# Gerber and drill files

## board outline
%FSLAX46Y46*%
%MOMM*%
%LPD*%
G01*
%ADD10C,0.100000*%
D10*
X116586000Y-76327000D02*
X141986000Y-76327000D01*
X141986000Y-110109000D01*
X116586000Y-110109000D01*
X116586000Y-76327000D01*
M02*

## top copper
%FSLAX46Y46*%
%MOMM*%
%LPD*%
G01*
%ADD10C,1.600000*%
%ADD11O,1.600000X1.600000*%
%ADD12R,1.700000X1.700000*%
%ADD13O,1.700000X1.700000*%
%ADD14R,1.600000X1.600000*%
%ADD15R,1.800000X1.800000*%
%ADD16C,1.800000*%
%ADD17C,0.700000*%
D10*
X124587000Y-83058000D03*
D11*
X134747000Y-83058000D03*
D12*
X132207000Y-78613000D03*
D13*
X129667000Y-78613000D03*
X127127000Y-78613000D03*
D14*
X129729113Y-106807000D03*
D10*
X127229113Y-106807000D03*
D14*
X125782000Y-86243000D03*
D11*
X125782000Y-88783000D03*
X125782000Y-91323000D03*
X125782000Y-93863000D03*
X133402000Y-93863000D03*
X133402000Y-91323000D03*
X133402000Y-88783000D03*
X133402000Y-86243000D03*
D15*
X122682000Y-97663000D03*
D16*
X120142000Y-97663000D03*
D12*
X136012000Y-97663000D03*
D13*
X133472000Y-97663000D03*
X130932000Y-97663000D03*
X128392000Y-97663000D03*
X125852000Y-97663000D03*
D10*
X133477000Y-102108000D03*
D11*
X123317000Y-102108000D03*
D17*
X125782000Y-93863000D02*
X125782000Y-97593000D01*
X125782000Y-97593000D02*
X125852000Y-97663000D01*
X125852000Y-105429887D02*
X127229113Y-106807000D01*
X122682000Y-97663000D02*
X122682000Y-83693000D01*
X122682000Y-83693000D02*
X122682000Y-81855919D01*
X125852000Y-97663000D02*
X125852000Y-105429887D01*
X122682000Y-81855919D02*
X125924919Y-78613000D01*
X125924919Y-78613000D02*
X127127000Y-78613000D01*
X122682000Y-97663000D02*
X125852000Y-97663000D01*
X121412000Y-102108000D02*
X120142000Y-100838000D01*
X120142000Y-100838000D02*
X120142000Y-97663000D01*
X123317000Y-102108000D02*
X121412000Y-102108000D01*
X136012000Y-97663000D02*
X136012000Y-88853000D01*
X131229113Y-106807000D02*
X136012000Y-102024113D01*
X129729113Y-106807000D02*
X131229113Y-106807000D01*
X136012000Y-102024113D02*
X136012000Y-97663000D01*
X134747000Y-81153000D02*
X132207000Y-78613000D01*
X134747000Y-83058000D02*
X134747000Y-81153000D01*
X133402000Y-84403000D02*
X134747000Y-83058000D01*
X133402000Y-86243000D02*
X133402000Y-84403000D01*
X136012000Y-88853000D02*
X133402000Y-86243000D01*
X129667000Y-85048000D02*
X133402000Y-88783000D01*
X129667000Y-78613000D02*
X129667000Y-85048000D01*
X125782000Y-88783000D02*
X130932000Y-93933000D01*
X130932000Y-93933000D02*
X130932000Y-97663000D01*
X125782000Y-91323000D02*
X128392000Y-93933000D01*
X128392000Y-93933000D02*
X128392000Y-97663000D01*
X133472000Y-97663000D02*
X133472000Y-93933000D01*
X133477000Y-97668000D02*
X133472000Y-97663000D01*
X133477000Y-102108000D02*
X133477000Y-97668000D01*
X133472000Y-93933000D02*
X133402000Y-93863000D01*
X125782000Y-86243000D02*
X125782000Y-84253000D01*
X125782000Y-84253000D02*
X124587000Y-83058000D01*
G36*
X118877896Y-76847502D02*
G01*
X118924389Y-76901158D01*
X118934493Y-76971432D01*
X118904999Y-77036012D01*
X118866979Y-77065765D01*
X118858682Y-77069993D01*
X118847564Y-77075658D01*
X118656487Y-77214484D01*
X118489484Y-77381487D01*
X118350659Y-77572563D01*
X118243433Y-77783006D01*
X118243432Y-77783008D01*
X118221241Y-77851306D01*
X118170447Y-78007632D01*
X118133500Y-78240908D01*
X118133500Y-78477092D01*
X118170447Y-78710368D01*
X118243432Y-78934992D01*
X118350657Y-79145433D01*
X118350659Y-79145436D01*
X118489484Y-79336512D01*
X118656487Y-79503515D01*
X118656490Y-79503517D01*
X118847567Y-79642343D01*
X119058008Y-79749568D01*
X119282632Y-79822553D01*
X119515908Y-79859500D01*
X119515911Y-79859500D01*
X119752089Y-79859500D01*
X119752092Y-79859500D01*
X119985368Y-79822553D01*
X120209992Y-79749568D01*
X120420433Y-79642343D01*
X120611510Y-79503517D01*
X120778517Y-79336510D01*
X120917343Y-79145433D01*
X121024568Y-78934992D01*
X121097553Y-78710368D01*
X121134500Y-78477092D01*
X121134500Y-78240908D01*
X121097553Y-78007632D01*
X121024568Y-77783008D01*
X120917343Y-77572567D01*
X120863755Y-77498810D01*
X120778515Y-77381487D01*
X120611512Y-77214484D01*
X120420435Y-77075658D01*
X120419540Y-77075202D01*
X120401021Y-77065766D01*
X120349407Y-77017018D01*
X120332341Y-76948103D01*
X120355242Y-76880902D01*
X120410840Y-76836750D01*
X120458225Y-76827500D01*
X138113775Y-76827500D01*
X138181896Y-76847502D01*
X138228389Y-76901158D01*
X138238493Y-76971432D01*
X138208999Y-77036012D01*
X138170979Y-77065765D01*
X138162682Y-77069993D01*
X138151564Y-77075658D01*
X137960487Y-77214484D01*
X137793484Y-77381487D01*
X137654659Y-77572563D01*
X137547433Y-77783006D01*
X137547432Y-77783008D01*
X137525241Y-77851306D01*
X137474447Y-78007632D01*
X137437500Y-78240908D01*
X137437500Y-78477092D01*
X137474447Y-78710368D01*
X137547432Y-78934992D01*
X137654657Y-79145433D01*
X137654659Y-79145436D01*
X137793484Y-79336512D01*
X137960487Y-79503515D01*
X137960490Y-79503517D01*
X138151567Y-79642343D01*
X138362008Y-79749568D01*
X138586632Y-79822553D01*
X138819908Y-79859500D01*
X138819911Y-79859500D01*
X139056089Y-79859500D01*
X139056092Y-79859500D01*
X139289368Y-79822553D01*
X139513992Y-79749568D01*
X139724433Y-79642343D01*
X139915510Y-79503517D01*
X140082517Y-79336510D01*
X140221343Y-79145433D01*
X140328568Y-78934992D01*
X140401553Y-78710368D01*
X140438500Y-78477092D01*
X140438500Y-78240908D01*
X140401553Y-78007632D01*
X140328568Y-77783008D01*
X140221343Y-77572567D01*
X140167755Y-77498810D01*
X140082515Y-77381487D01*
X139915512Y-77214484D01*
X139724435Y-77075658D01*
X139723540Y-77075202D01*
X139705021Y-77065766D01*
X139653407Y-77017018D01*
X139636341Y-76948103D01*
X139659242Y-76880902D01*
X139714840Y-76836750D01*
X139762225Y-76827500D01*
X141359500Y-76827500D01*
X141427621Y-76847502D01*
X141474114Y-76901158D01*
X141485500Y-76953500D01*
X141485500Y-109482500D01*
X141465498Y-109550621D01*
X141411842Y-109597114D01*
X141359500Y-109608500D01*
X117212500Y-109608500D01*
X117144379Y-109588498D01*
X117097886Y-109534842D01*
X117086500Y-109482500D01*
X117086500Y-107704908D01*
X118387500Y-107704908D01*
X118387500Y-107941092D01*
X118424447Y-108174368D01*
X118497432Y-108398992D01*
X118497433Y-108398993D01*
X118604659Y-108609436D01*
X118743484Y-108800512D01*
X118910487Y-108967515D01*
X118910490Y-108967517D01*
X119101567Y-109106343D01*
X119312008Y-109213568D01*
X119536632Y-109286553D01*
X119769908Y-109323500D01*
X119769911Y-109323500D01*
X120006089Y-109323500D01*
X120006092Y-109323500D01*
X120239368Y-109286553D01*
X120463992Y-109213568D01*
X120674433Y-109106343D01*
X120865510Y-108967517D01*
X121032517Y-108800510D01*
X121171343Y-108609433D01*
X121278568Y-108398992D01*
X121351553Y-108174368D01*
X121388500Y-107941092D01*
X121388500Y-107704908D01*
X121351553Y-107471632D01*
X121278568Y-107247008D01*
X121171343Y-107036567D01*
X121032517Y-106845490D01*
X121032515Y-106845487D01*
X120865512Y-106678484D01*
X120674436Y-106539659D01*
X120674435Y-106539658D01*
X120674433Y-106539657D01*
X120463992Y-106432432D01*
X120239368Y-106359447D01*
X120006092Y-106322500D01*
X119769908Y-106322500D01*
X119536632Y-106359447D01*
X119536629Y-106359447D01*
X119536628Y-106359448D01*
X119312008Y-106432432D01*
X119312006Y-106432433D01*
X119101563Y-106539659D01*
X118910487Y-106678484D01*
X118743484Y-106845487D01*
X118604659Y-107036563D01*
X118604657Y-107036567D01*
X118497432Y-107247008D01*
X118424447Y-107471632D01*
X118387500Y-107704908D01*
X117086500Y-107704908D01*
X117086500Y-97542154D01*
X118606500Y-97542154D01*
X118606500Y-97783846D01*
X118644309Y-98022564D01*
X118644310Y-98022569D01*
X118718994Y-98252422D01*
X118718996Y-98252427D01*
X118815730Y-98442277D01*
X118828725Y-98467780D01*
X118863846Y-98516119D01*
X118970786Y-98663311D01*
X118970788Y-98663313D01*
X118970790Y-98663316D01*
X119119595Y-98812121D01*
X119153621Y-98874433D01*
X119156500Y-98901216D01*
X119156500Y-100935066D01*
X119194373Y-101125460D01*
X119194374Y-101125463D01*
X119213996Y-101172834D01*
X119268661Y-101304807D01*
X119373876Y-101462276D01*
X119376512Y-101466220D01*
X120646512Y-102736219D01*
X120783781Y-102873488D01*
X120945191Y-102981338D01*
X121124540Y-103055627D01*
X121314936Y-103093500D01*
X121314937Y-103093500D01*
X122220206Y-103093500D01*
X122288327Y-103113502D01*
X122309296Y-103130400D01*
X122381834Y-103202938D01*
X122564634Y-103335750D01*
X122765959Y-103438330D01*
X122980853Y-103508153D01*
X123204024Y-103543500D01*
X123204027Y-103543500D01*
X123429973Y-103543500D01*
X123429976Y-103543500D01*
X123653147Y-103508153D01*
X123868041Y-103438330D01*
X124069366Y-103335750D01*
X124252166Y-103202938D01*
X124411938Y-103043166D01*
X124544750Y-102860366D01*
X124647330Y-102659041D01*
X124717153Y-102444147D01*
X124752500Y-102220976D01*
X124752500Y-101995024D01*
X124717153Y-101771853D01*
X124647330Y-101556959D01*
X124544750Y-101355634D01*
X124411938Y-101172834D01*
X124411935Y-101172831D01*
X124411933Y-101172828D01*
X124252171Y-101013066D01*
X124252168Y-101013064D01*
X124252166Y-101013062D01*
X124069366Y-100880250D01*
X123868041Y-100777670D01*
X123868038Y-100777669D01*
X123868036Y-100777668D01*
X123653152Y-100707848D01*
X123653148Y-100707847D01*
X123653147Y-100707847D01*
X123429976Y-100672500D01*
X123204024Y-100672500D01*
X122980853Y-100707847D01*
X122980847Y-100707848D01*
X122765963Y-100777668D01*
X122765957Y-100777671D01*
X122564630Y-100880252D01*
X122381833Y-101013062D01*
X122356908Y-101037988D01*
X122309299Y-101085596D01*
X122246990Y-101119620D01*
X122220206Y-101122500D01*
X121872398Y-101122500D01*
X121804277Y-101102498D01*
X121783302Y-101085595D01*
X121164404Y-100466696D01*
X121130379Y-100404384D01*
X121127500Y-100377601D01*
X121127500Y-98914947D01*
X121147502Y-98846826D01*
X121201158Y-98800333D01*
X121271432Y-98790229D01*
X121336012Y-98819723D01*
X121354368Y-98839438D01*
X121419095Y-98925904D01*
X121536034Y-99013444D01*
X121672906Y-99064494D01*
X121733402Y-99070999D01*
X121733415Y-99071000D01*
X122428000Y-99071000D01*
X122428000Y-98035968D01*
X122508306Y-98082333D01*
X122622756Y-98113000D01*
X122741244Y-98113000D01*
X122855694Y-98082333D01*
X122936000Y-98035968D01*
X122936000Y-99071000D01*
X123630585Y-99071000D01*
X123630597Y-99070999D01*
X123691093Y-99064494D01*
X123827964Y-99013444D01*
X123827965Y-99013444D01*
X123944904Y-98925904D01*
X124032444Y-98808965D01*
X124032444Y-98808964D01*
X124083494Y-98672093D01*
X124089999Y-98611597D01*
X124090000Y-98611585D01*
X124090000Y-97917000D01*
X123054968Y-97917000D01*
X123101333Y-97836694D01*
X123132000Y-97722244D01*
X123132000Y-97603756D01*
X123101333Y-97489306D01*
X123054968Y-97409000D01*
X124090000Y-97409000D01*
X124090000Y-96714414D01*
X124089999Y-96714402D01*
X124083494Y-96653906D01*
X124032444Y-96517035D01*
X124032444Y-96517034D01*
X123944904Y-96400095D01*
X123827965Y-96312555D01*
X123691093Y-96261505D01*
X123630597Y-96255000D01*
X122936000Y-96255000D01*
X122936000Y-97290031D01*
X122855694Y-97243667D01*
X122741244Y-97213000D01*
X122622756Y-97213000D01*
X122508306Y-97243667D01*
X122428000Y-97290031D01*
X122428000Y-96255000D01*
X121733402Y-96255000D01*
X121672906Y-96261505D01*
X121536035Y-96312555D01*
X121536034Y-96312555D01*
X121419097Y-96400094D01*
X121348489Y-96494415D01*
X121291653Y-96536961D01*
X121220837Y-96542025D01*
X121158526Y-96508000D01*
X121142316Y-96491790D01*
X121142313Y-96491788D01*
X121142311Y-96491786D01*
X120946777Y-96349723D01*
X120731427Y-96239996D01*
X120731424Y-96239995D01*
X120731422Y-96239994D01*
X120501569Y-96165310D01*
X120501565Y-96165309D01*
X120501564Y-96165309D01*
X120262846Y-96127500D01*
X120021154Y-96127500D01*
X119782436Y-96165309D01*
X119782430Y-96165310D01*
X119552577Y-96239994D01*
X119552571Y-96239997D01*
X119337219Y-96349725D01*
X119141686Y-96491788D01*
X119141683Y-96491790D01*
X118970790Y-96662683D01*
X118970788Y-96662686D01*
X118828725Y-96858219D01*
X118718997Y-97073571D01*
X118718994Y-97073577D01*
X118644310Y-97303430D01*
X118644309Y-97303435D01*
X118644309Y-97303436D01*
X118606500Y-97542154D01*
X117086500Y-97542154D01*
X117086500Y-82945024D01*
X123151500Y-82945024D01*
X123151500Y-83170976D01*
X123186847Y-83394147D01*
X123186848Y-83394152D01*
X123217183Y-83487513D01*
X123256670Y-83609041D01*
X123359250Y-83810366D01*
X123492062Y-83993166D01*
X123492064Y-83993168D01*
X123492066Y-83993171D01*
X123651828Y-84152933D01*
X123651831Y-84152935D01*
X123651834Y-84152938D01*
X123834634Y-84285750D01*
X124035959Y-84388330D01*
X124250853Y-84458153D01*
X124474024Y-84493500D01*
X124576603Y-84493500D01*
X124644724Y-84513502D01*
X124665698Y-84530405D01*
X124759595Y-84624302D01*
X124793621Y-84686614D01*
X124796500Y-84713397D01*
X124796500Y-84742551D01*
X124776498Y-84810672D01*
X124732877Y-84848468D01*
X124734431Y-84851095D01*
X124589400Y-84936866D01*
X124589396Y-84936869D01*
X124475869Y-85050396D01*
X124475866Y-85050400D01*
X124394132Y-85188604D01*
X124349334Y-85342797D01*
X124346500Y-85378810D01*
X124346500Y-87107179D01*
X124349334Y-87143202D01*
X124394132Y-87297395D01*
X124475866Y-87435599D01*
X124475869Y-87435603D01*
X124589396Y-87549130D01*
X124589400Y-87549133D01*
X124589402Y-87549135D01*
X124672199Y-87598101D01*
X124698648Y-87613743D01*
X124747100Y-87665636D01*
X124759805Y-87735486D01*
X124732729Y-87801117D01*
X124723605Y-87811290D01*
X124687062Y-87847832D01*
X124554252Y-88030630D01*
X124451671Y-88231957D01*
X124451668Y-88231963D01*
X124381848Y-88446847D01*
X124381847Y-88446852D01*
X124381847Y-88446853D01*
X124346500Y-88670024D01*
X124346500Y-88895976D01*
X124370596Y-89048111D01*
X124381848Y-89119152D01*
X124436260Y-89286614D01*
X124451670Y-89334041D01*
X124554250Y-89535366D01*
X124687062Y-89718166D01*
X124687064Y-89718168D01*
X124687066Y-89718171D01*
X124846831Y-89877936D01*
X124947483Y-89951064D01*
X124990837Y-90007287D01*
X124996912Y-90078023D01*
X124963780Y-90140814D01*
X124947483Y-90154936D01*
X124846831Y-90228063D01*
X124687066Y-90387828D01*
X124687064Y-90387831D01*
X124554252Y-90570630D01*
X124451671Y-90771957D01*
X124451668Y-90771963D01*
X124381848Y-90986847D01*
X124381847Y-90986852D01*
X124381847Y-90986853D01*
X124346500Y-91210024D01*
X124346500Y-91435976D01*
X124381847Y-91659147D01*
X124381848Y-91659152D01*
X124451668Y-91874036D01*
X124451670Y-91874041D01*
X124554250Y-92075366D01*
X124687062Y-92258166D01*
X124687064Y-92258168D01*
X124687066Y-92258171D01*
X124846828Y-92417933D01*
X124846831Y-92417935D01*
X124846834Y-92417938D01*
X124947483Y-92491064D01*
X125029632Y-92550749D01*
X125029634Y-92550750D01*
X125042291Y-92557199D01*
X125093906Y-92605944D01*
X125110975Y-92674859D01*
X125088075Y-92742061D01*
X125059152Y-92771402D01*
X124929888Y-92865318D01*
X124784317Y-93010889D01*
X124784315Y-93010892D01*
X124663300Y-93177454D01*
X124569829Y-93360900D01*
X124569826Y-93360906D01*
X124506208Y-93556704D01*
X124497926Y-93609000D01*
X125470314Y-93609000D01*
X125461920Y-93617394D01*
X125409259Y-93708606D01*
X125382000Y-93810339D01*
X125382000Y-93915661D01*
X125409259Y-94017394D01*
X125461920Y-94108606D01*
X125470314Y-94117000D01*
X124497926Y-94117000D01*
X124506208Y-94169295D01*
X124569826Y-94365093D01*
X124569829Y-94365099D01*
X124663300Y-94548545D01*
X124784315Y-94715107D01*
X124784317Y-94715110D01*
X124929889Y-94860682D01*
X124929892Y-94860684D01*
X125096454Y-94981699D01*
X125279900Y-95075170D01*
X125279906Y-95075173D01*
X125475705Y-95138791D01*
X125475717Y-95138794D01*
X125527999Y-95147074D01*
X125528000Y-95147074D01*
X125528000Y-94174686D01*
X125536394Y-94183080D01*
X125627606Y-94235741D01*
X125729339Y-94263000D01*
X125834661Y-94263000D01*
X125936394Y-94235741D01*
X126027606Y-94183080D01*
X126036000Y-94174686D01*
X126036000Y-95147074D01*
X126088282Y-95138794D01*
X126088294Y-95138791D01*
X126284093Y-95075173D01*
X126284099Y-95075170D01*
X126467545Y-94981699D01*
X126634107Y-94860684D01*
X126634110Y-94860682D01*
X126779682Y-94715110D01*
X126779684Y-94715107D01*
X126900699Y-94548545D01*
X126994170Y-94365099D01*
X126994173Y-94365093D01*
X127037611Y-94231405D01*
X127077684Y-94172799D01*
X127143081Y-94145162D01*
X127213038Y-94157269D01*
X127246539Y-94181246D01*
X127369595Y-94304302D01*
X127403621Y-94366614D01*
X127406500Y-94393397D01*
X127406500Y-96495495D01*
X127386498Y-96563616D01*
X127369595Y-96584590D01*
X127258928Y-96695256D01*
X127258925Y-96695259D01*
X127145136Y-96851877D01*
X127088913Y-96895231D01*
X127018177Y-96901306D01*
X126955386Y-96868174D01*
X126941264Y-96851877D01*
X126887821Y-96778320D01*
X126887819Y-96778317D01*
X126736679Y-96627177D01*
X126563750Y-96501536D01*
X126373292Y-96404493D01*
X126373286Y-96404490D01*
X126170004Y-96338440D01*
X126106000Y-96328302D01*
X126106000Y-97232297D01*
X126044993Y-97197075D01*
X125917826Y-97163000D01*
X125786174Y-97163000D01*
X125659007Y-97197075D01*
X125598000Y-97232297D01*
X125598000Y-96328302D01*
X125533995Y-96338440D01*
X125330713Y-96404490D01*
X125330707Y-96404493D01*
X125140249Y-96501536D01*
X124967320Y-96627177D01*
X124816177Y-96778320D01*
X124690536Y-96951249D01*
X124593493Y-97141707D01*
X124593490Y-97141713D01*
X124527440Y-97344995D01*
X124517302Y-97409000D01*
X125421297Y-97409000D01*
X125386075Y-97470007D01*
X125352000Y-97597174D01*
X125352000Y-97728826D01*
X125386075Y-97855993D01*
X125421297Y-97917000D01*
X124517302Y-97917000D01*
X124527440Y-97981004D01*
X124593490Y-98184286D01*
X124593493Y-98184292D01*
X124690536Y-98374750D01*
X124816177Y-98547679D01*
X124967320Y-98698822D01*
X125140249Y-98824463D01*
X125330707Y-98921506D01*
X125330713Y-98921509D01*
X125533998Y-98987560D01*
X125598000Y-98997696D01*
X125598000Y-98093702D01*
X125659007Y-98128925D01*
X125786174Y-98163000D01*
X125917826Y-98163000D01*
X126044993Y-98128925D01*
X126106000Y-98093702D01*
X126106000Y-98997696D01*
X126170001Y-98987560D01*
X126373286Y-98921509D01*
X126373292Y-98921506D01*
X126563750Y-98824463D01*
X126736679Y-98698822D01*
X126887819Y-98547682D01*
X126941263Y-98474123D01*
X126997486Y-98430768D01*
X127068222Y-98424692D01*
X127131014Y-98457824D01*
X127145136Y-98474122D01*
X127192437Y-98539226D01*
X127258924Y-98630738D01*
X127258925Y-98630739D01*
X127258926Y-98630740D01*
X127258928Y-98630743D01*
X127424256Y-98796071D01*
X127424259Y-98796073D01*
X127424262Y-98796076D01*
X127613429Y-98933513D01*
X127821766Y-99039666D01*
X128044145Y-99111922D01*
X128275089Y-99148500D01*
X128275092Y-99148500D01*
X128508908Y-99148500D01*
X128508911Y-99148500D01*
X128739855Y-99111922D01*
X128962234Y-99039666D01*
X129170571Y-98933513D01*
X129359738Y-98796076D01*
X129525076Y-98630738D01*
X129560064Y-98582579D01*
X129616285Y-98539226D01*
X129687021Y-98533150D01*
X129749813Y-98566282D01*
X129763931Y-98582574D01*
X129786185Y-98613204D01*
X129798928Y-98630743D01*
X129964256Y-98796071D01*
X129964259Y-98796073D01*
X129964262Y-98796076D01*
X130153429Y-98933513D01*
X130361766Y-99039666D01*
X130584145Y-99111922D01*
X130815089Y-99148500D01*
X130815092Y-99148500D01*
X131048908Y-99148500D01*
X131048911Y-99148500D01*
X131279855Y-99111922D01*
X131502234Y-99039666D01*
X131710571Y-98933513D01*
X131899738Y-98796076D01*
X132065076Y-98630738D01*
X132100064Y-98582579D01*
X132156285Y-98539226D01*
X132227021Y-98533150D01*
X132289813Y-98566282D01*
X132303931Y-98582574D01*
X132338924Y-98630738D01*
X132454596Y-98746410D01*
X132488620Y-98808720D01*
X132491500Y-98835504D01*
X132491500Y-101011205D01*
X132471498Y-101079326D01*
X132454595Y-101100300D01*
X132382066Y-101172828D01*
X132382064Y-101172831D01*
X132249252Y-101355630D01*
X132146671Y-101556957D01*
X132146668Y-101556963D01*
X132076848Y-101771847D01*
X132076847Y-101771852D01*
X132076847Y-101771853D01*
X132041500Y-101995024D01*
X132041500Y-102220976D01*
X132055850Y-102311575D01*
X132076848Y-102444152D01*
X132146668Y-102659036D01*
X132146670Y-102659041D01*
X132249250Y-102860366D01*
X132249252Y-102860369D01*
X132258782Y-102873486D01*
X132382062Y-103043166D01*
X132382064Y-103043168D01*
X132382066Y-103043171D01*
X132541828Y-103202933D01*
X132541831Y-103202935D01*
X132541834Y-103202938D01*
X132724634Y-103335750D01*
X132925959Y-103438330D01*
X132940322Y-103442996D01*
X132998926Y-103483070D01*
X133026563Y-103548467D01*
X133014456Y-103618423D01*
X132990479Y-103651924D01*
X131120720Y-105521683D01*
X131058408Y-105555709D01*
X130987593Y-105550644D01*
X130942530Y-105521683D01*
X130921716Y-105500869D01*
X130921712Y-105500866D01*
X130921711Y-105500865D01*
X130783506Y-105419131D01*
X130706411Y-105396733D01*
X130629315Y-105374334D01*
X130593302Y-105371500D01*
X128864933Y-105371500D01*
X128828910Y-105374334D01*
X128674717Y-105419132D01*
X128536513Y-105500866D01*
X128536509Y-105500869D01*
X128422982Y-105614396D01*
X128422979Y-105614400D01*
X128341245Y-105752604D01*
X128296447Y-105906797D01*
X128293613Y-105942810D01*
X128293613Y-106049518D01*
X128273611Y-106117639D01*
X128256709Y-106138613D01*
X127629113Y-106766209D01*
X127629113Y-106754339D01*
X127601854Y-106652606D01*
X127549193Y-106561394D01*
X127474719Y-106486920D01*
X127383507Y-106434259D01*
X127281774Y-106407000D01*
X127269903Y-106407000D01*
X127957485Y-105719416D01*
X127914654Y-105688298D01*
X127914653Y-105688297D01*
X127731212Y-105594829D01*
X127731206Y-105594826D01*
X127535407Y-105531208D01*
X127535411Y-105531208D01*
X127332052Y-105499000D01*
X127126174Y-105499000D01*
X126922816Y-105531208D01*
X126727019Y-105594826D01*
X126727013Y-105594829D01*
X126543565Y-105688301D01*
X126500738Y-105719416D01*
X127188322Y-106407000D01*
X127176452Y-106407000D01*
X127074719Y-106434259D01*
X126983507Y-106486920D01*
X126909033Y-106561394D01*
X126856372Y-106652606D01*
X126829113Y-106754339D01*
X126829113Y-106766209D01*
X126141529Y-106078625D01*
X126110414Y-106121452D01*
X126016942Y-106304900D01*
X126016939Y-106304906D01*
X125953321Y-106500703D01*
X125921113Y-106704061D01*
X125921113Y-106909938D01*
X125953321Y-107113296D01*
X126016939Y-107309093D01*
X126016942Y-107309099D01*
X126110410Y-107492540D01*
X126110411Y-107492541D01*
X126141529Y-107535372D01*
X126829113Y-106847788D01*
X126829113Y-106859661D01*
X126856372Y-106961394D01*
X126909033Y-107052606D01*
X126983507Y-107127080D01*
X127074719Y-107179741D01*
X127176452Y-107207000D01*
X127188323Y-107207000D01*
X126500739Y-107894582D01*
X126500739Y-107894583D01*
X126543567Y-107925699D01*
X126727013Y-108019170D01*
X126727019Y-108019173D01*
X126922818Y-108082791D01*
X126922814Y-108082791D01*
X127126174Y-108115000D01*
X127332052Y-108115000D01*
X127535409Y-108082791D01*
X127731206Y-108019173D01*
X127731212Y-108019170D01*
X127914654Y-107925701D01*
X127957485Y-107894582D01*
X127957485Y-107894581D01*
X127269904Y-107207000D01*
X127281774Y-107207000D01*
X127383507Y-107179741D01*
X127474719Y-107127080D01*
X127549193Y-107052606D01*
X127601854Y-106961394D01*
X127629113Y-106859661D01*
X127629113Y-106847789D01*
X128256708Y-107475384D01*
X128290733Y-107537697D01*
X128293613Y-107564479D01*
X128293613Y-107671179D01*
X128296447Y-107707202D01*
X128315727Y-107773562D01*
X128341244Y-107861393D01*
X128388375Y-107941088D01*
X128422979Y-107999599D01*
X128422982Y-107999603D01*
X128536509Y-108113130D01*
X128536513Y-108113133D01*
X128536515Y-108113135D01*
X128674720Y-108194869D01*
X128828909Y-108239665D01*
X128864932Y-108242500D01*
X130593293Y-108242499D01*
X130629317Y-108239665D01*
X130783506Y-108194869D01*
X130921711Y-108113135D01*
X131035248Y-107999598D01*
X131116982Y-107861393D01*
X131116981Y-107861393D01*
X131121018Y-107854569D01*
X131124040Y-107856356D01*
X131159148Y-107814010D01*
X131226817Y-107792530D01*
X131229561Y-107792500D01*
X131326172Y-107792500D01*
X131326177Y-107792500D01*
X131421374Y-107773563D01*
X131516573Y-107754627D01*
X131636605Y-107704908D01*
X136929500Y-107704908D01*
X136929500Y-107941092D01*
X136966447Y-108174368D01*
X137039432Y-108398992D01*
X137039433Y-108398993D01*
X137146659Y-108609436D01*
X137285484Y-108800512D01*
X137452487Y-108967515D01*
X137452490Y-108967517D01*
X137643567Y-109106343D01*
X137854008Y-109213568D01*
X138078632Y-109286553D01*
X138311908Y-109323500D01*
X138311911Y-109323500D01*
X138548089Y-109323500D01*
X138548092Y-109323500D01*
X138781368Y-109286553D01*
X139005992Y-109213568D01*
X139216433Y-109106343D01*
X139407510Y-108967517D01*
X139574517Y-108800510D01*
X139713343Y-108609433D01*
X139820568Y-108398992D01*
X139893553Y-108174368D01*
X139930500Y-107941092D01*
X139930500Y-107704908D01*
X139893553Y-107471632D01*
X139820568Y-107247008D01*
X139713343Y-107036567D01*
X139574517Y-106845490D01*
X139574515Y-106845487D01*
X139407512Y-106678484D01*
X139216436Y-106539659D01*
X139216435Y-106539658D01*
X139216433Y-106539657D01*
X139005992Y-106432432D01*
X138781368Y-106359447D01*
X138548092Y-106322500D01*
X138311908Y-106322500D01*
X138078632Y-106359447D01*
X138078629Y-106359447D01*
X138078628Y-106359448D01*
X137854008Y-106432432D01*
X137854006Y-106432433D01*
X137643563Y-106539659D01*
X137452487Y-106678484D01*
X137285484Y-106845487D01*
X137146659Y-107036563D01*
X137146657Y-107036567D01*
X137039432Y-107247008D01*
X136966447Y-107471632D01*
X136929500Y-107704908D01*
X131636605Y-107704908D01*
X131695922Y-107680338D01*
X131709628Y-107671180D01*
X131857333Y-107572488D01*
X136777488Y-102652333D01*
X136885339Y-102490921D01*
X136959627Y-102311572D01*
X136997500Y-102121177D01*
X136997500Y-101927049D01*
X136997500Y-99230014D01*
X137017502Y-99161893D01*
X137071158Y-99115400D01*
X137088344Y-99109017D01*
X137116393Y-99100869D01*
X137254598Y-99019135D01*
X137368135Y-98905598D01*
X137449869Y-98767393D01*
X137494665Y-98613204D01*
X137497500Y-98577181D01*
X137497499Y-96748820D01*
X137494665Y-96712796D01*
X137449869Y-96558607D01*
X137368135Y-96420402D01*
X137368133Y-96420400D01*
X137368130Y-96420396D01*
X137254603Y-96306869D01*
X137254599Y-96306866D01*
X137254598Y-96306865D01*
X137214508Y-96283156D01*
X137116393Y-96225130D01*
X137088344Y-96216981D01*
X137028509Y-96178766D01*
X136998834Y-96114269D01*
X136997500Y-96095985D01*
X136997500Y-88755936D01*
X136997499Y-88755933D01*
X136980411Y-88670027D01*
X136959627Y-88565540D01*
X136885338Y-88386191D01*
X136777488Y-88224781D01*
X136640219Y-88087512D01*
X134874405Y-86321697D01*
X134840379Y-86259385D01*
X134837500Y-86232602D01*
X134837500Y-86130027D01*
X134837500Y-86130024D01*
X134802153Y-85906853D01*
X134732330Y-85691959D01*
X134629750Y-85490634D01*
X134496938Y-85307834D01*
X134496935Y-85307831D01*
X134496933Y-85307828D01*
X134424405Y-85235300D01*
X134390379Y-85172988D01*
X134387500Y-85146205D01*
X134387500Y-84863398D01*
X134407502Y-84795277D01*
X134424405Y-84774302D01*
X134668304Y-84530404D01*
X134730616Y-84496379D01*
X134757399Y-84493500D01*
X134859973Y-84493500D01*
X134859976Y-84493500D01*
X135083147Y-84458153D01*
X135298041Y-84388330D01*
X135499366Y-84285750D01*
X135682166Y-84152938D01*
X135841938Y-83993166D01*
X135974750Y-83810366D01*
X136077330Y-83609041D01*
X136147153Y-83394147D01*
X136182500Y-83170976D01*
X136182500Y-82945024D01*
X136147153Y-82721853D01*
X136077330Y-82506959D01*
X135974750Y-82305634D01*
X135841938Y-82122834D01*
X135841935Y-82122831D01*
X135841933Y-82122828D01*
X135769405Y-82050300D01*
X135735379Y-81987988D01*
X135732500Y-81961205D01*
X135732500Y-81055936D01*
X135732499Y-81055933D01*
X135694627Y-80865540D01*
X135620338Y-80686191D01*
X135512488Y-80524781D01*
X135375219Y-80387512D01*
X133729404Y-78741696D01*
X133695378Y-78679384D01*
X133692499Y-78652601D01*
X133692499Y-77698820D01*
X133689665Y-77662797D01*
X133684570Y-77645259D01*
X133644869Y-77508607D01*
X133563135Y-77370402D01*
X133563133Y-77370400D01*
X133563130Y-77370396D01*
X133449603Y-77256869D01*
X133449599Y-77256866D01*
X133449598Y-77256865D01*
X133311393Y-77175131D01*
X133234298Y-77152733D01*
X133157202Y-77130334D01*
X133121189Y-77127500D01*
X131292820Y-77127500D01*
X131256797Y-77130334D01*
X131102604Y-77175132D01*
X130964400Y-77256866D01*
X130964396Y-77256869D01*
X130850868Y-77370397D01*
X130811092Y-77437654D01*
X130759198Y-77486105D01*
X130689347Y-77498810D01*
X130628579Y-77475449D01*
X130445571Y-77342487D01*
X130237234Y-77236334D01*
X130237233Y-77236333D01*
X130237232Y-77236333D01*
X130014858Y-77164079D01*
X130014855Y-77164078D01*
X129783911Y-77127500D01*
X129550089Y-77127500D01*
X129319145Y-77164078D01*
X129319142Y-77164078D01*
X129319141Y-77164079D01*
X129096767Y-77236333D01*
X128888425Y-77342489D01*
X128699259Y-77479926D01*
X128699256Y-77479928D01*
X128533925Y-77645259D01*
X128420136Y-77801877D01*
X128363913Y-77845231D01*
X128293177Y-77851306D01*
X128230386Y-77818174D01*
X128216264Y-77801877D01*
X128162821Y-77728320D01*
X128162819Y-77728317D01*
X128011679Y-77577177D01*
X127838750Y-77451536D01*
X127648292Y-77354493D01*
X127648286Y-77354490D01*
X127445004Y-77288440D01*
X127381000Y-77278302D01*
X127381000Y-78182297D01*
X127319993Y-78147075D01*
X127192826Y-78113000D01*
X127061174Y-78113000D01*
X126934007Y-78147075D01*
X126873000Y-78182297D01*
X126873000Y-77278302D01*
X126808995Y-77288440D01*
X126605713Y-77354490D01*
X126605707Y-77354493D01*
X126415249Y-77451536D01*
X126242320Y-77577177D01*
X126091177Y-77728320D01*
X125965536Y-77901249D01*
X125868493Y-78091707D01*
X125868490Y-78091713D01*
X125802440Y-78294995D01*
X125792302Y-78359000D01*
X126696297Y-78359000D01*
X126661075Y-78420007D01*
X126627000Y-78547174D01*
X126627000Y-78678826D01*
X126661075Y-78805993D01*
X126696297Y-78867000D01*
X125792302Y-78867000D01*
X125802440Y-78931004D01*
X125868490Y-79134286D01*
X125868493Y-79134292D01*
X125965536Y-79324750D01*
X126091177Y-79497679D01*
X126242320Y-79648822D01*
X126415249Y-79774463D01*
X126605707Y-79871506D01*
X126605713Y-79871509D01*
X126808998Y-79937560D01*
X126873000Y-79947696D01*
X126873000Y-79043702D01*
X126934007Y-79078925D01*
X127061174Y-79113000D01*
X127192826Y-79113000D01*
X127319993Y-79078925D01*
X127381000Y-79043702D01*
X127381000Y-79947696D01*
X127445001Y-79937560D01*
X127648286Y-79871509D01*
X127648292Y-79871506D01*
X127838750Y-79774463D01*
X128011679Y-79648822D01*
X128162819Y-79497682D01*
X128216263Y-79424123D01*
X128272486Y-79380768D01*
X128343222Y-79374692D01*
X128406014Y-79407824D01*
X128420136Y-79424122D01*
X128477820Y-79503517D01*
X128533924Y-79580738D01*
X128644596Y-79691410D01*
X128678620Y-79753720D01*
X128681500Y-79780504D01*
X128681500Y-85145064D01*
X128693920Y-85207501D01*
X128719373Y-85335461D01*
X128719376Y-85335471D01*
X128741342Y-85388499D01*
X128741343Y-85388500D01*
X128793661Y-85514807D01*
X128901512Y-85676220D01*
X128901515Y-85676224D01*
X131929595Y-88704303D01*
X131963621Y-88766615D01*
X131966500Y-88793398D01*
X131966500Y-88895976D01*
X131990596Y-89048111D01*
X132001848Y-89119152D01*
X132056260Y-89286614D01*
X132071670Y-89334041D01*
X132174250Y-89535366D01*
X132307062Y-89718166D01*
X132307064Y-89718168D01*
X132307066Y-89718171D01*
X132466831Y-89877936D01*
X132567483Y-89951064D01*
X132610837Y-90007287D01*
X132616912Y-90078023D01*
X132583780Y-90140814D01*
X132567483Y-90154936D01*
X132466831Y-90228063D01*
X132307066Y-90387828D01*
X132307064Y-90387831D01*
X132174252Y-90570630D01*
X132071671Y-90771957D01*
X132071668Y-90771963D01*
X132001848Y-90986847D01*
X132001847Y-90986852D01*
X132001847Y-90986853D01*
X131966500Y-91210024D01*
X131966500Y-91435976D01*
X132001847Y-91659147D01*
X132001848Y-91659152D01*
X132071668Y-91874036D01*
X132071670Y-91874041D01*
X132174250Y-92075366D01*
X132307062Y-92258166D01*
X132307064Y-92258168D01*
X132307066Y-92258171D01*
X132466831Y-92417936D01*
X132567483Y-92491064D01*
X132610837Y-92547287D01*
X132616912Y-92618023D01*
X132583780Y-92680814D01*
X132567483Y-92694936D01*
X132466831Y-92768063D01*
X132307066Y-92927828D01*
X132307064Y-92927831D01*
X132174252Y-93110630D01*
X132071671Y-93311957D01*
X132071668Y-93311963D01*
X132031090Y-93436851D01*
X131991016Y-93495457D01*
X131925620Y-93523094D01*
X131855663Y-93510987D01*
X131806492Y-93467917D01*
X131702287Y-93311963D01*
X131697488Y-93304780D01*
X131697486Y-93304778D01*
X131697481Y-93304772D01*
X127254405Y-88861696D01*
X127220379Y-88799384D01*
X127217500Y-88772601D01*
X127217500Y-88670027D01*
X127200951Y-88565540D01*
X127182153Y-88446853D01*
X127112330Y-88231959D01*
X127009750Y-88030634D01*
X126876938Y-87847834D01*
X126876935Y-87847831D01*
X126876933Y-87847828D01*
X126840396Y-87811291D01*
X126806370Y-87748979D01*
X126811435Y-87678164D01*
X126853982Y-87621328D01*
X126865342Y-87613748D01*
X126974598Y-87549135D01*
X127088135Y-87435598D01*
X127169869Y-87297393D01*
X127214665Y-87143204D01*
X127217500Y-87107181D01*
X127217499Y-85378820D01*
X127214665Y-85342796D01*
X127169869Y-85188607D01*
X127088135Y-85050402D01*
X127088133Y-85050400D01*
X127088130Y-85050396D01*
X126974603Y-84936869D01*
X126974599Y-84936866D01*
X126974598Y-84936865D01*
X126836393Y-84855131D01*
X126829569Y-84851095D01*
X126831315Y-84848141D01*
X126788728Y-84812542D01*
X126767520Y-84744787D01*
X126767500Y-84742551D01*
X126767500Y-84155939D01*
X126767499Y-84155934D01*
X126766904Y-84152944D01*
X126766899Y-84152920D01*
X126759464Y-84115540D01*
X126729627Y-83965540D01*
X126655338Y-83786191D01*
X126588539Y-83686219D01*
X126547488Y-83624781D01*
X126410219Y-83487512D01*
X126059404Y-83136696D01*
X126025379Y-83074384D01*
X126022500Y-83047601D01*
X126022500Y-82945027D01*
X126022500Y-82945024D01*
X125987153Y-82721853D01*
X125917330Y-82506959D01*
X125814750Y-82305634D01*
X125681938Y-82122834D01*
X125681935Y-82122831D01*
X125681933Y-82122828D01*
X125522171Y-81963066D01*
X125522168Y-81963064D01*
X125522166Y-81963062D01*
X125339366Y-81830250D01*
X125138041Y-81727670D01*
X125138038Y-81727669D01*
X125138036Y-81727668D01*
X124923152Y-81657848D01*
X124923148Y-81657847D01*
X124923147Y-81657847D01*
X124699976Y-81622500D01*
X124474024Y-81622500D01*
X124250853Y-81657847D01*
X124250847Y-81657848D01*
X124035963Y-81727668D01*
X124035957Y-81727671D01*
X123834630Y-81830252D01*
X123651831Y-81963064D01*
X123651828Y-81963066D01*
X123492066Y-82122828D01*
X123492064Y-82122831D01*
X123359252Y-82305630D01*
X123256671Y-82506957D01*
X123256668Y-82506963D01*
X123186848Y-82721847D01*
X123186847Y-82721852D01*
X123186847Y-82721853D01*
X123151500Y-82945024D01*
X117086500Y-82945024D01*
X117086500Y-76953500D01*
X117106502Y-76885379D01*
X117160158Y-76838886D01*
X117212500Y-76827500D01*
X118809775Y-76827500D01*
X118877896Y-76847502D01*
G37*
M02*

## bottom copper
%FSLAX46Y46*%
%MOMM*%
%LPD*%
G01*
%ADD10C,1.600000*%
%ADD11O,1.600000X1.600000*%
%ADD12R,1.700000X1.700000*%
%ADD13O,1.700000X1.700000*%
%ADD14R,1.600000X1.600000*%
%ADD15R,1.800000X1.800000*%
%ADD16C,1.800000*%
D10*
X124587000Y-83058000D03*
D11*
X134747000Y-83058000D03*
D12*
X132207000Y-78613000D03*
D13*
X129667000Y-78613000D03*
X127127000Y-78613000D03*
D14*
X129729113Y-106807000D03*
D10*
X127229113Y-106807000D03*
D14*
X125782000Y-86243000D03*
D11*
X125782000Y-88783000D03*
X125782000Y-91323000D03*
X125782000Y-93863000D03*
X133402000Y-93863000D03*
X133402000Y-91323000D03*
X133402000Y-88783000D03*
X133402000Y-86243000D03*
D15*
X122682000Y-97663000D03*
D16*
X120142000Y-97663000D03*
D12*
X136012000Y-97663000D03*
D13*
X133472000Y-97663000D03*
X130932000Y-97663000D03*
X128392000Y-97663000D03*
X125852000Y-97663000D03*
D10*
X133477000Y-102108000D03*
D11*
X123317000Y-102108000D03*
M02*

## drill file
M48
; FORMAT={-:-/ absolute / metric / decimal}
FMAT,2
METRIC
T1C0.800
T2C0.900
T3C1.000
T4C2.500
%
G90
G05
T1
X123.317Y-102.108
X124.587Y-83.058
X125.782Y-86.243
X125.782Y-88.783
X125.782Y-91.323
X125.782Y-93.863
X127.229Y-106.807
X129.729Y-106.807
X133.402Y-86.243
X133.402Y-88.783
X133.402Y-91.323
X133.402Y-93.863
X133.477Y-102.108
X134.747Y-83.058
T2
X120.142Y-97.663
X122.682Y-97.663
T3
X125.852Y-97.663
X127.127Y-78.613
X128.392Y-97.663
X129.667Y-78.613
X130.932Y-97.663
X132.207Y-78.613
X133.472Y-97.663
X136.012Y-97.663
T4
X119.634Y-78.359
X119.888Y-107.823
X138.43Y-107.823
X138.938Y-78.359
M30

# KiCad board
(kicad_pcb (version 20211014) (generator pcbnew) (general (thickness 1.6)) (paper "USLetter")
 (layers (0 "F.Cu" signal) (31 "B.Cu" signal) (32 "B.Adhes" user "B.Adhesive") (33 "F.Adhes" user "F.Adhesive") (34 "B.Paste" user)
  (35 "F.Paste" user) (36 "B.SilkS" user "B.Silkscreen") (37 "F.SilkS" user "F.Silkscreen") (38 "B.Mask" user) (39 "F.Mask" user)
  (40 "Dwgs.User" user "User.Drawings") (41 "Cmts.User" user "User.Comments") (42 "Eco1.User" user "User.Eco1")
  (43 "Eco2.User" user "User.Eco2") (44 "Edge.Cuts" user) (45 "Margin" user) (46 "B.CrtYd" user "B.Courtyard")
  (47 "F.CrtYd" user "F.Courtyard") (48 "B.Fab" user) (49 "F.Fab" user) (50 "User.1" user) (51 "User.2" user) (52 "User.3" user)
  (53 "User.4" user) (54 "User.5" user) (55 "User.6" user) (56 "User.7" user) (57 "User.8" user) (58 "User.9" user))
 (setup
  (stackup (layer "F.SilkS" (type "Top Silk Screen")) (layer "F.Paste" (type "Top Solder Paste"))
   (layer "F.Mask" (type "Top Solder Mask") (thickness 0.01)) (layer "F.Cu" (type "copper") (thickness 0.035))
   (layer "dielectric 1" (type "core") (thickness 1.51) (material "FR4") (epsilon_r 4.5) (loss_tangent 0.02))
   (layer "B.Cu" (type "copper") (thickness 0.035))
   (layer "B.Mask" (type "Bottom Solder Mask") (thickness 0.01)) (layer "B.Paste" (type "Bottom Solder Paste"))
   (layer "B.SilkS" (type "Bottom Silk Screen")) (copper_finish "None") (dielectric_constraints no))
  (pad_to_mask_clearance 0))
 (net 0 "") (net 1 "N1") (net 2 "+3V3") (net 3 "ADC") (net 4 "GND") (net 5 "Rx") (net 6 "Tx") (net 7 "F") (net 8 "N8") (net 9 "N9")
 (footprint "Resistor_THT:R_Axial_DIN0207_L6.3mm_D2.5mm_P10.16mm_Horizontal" (layer "F.Cu") (at 124.587 83.058)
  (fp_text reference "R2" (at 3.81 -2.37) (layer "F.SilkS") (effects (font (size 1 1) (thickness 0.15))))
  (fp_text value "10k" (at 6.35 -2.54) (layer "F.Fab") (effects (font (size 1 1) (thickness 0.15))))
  (pad "1" thru_hole circle locked (at 0 0) (size 1.6 1.6) (drill 0.8) (layers *.Cu *.Mask) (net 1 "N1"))
  (pad "2" thru_hole oval locked (at 10.16 0) (size 1.6 1.6) (drill 0.8) (layers *.Cu *.Mask) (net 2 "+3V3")))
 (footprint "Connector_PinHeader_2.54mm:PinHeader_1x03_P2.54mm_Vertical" (layer "F.Cu") (at 132.207 78.613 -90)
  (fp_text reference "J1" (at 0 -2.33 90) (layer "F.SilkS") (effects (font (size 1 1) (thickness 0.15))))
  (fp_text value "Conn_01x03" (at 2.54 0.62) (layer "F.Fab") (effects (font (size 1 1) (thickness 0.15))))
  (pad "1" thru_hole rect locked (at 0 0 270) (size 1.7 1.7) (drill 1) (layers *.Cu *.Mask) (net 2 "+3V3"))
  (pad "2" thru_hole oval locked (at 0 2.54 270) (size 1.7 1.7) (drill 1) (layers *.Cu *.Mask) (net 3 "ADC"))
  (pad "3" thru_hole oval locked (at 0 5.08 270) (size 1.7 1.7) (drill 1) (layers *.Cu *.Mask) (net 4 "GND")))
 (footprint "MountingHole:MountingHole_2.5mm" (layer "F.Cu") (at 138.43 107.823)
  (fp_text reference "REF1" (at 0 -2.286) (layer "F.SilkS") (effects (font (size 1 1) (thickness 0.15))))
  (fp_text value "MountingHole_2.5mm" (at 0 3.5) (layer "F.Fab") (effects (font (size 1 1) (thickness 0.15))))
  (pad "" np_thru_hole circle locked (at 0 0) (size 2.5 2.5) (drill 2.5) (layers *.Cu *.Mask)))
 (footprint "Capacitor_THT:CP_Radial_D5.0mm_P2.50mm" (layer "F.Cu") (at 129.729113 106.807 180)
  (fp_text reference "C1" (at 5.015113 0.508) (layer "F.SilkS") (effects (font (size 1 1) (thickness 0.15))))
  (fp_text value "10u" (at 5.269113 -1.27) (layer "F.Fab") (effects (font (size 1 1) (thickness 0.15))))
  (pad "1" thru_hole rect locked (at 0 0 180) (size 1.6 1.6) (drill 0.8) (layers *.Cu *.Mask) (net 2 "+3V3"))
  (pad "2" thru_hole circle locked (at 2.5 0 180) (size 1.6 1.6) (drill 0.8) (layers *.Cu *.Mask) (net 4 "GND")))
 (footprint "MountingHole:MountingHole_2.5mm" (layer "F.Cu") (at 138.938 78.359)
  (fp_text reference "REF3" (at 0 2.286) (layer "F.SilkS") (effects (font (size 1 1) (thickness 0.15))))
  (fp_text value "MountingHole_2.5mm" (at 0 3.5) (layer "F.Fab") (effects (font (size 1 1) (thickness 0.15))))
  (pad "" np_thru_hole circle locked (at 0 0) (size 2.5 2.5) (drill 2.5) (layers *.Cu *.Mask)))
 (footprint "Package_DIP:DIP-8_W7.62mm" (layer "F.Cu") (at 125.782 86.243)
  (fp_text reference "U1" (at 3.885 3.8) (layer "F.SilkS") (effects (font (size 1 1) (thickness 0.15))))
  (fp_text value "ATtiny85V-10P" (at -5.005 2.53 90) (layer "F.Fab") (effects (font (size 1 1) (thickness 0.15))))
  (pad "1" thru_hole rect locked (at 0 0) (size 1.6 1.6) (drill 0.8) (layers *.Cu *.Mask) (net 1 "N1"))
  (pad "2" thru_hole oval locked (at 0 2.54) (size 1.6 1.6) (drill 0.8) (layers *.Cu *.Mask) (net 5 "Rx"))
  (pad "3" thru_hole oval locked (at 0 5.08) (size 1.6 1.6) (drill 0.8) (layers *.Cu *.Mask) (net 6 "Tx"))
  (pad "4" thru_hole oval locked (at 0 7.62) (size 1.6 1.6) (drill 0.8) (layers *.Cu *.Mask) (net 4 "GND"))
  (pad "5" thru_hole oval locked (at 7.62 7.62) (size 1.6 1.6) (drill 0.8) (layers *.Cu *.Mask) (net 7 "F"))
  (pad "6" thru_hole oval locked (at 7.62 5.08) (size 1.6 1.6) (drill 0.8) (layers *.Cu *.Mask) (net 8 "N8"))
  (pad "7" thru_hole oval locked (at 7.62 2.54) (size 1.6 1.6) (drill 0.8) (layers *.Cu *.Mask) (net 3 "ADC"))
  (pad "8" thru_hole oval locked (at 7.62 0) (size 1.6 1.6) (drill 0.8) (layers *.Cu *.Mask) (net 2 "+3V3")))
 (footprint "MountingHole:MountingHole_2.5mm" (layer "F.Cu") (at 119.888 107.823)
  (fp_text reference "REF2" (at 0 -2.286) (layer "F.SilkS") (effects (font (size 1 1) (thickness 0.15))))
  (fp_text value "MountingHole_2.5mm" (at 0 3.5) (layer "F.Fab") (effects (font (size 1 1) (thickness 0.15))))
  (pad "" np_thru_hole circle locked (at 0 0) (size 2.5 2.5) (drill 2.5) (layers *.Cu *.Mask)))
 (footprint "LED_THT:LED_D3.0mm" (layer "F.Cu") (at 122.682 97.663 180)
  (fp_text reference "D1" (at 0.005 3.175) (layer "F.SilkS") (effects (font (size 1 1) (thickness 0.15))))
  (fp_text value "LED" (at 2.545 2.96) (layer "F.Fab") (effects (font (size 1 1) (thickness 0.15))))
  (pad "1" thru_hole rect locked (at 0 0 180) (size 1.8 1.8) (drill 0.9) (layers *.Cu *.Mask) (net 4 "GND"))
  (pad "2" thru_hole circle locked (at 2.54 0 180) (size 1.8 1.8) (drill 0.9) (layers *.Cu *.Mask) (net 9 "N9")))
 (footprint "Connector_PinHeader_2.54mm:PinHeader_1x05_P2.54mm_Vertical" (layer "F.Cu") (at 136.012 97.663 -90)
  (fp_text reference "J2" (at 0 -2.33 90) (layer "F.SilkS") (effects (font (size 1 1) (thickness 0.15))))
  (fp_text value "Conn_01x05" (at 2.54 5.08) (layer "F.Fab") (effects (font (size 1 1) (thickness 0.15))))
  (pad "1" thru_hole rect locked (at 0 0 270) (size 1.7 1.7) (drill 1) (layers *.Cu *.Mask) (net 2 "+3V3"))
  (pad "2" thru_hole oval locked (at 0 2.54 270) (size 1.7 1.7) (drill 1) (layers *.Cu *.Mask) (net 7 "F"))
  (pad "3" thru_hole oval locked (at 0 5.08 270) (size 1.7 1.7) (drill 1) (layers *.Cu *.Mask) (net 5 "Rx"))
  (pad "4" thru_hole oval locked (at 0 7.62 270) (size 1.7 1.7) (drill 1) (layers *.Cu *.Mask) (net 6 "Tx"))
  (pad "5" thru_hole oval locked (at 0 10.16 270) (size 1.7 1.7) (drill 1) (layers *.Cu *.Mask) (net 4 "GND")))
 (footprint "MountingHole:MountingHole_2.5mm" (layer "F.Cu") (at 119.634 78.359)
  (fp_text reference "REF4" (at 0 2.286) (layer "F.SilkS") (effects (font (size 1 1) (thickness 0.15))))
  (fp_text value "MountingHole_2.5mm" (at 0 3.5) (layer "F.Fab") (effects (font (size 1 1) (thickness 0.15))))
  (pad "" np_thru_hole circle locked (at 0 0) (size 2.5 2.5) (drill 2.5) (layers *.Cu *.Mask)))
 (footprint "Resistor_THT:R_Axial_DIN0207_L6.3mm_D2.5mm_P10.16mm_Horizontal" (layer "F.Cu") (at 133.477 102.108 180)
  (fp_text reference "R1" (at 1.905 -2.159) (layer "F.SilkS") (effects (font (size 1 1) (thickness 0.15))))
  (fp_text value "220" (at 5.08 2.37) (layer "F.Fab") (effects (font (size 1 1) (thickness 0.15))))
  (pad "1" thru_hole circle locked (at 0 0 180) (size 1.6 1.6) (drill 0.8) (layers *.Cu *.Mask) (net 7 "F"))
  (pad "2" thru_hole oval locked (at 10.16 0 180) (size 1.6 1.6) (drill 0.8) (layers *.Cu *.Mask) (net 9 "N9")))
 (gr_rect (start 116.586 76.327) (end 141.986 110.109) (layer "Edge.Cuts") (width 0.1) (fill none))
 (segment (start 125.782 93.863) (end 125.782 97.593) (width 0.7) (layer "F.Cu") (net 4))
 (segment (start 125.782 97.593) (end 125.852 97.663) (width 0.7) (layer "F.Cu") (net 4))
 (segment (start 125.852 105.429887) (end 127.229113 106.807) (width 0.7) (layer "F.Cu") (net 4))
 (segment (start 122.682 97.663) (end 122.682 83.693) (width 0.7) (layer "F.Cu") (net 4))
 (segment (start 122.682 83.693) (end 122.682 81.855919) (width 0.7) (layer "F.Cu") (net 4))
 (segment (start 125.852 97.663) (end 125.852 105.429887) (width 0.7) (layer "F.Cu") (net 4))
 (segment (start 122.682 81.855919) (end 125.924919 78.613) (width 0.7) (layer "F.Cu") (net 4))
 (segment (start 125.924919 78.613) (end 127.127 78.613) (width 0.7) (layer "F.Cu") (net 4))
 (segment (start 122.682 97.663) (end 125.852 97.663) (width 0.7) (layer "F.Cu") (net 4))
 (segment (start 121.412 102.108) (end 120.142 100.838) (width 0.7) (layer "F.Cu") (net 9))
 (segment (start 120.142 100.838) (end 120.142 97.663) (width 0.7) (layer "F.Cu") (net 9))
 (segment (start 123.317 102.108) (end 121.412 102.108) (width 0.7) (layer "F.Cu") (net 9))
 (segment (start 136.012 97.663) (end 136.012 88.853) (width 0.7) (layer "F.Cu") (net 2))
 (segment (start 131.229113 106.807) (end 136.012 102.024113) (width 0.7) (layer "F.Cu") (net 2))
 (segment (start 129.729113 106.807) (end 131.229113 106.807) (width 0.7) (layer "F.Cu") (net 2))
 (segment (start 136.012 102.024113) (end 136.012 97.663) (width 0.7) (layer "F.Cu") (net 2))
 (segment (start 134.747 81.153) (end 132.207 78.613) (width 0.7) (layer "F.Cu") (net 2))
 (segment (start 134.747 83.058) (end 134.747 81.153) (width 0.7) (layer "F.Cu") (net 2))
 (segment (start 133.402 84.403) (end 134.747 83.058) (width 0.7) (layer "F.Cu") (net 2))
 (segment (start 133.402 86.243) (end 133.402 84.403) (width 0.7) (layer "F.Cu") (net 2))
 (segment (start 136.012 88.853) (end 133.402 86.243) (width 0.7) (layer "F.Cu") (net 2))
 (segment (start 129.667 85.048) (end 133.402 88.783) (width 0.7) (layer "F.Cu") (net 3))
 (segment (start 129.667 78.613) (end 129.667 85.048) (width 0.7) (layer "F.Cu") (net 3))
 (segment (start 125.782 88.783) (end 130.932 93.933) (width 0.7) (layer "F.Cu") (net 5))
 (segment (start 130.932 93.933) (end 130.932 97.663) (width 0.7) (layer "F.Cu") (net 5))
 (segment (start 125.782 91.323) (end 128.392 93.933) (width 0.7) (layer "F.Cu") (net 6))
 (segment (start 128.392 93.933) (end 128.392 97.663) (width 0.7) (layer "F.Cu") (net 6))
 (segment (start 133.472 97.663) (end 133.472 93.933) (width 0.7) (layer "F.Cu") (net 7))
 (segment (start 133.477 97.668) (end 133.472 97.663) (width 0.7) (layer "F.Cu") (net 7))
 (segment (start 133.477 102.108) (end 133.477 97.668) (width 0.7) (layer "F.Cu") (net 7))
 (segment (start 133.472 93.933) (end 133.402 93.863) (width 0.7) (layer "F.Cu") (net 7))
 (segment (start 125.782 86.243) (end 125.782 84.253) (width 0.7) (layer "F.Cu") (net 1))
 (segment (start 125.782 84.253) (end 124.587 83.058) (width 0.7) (layer "F.Cu") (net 1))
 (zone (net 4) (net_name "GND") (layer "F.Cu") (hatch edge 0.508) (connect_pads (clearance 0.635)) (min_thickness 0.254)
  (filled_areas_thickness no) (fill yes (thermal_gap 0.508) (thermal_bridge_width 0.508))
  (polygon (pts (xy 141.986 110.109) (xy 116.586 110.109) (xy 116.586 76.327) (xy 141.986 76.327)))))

